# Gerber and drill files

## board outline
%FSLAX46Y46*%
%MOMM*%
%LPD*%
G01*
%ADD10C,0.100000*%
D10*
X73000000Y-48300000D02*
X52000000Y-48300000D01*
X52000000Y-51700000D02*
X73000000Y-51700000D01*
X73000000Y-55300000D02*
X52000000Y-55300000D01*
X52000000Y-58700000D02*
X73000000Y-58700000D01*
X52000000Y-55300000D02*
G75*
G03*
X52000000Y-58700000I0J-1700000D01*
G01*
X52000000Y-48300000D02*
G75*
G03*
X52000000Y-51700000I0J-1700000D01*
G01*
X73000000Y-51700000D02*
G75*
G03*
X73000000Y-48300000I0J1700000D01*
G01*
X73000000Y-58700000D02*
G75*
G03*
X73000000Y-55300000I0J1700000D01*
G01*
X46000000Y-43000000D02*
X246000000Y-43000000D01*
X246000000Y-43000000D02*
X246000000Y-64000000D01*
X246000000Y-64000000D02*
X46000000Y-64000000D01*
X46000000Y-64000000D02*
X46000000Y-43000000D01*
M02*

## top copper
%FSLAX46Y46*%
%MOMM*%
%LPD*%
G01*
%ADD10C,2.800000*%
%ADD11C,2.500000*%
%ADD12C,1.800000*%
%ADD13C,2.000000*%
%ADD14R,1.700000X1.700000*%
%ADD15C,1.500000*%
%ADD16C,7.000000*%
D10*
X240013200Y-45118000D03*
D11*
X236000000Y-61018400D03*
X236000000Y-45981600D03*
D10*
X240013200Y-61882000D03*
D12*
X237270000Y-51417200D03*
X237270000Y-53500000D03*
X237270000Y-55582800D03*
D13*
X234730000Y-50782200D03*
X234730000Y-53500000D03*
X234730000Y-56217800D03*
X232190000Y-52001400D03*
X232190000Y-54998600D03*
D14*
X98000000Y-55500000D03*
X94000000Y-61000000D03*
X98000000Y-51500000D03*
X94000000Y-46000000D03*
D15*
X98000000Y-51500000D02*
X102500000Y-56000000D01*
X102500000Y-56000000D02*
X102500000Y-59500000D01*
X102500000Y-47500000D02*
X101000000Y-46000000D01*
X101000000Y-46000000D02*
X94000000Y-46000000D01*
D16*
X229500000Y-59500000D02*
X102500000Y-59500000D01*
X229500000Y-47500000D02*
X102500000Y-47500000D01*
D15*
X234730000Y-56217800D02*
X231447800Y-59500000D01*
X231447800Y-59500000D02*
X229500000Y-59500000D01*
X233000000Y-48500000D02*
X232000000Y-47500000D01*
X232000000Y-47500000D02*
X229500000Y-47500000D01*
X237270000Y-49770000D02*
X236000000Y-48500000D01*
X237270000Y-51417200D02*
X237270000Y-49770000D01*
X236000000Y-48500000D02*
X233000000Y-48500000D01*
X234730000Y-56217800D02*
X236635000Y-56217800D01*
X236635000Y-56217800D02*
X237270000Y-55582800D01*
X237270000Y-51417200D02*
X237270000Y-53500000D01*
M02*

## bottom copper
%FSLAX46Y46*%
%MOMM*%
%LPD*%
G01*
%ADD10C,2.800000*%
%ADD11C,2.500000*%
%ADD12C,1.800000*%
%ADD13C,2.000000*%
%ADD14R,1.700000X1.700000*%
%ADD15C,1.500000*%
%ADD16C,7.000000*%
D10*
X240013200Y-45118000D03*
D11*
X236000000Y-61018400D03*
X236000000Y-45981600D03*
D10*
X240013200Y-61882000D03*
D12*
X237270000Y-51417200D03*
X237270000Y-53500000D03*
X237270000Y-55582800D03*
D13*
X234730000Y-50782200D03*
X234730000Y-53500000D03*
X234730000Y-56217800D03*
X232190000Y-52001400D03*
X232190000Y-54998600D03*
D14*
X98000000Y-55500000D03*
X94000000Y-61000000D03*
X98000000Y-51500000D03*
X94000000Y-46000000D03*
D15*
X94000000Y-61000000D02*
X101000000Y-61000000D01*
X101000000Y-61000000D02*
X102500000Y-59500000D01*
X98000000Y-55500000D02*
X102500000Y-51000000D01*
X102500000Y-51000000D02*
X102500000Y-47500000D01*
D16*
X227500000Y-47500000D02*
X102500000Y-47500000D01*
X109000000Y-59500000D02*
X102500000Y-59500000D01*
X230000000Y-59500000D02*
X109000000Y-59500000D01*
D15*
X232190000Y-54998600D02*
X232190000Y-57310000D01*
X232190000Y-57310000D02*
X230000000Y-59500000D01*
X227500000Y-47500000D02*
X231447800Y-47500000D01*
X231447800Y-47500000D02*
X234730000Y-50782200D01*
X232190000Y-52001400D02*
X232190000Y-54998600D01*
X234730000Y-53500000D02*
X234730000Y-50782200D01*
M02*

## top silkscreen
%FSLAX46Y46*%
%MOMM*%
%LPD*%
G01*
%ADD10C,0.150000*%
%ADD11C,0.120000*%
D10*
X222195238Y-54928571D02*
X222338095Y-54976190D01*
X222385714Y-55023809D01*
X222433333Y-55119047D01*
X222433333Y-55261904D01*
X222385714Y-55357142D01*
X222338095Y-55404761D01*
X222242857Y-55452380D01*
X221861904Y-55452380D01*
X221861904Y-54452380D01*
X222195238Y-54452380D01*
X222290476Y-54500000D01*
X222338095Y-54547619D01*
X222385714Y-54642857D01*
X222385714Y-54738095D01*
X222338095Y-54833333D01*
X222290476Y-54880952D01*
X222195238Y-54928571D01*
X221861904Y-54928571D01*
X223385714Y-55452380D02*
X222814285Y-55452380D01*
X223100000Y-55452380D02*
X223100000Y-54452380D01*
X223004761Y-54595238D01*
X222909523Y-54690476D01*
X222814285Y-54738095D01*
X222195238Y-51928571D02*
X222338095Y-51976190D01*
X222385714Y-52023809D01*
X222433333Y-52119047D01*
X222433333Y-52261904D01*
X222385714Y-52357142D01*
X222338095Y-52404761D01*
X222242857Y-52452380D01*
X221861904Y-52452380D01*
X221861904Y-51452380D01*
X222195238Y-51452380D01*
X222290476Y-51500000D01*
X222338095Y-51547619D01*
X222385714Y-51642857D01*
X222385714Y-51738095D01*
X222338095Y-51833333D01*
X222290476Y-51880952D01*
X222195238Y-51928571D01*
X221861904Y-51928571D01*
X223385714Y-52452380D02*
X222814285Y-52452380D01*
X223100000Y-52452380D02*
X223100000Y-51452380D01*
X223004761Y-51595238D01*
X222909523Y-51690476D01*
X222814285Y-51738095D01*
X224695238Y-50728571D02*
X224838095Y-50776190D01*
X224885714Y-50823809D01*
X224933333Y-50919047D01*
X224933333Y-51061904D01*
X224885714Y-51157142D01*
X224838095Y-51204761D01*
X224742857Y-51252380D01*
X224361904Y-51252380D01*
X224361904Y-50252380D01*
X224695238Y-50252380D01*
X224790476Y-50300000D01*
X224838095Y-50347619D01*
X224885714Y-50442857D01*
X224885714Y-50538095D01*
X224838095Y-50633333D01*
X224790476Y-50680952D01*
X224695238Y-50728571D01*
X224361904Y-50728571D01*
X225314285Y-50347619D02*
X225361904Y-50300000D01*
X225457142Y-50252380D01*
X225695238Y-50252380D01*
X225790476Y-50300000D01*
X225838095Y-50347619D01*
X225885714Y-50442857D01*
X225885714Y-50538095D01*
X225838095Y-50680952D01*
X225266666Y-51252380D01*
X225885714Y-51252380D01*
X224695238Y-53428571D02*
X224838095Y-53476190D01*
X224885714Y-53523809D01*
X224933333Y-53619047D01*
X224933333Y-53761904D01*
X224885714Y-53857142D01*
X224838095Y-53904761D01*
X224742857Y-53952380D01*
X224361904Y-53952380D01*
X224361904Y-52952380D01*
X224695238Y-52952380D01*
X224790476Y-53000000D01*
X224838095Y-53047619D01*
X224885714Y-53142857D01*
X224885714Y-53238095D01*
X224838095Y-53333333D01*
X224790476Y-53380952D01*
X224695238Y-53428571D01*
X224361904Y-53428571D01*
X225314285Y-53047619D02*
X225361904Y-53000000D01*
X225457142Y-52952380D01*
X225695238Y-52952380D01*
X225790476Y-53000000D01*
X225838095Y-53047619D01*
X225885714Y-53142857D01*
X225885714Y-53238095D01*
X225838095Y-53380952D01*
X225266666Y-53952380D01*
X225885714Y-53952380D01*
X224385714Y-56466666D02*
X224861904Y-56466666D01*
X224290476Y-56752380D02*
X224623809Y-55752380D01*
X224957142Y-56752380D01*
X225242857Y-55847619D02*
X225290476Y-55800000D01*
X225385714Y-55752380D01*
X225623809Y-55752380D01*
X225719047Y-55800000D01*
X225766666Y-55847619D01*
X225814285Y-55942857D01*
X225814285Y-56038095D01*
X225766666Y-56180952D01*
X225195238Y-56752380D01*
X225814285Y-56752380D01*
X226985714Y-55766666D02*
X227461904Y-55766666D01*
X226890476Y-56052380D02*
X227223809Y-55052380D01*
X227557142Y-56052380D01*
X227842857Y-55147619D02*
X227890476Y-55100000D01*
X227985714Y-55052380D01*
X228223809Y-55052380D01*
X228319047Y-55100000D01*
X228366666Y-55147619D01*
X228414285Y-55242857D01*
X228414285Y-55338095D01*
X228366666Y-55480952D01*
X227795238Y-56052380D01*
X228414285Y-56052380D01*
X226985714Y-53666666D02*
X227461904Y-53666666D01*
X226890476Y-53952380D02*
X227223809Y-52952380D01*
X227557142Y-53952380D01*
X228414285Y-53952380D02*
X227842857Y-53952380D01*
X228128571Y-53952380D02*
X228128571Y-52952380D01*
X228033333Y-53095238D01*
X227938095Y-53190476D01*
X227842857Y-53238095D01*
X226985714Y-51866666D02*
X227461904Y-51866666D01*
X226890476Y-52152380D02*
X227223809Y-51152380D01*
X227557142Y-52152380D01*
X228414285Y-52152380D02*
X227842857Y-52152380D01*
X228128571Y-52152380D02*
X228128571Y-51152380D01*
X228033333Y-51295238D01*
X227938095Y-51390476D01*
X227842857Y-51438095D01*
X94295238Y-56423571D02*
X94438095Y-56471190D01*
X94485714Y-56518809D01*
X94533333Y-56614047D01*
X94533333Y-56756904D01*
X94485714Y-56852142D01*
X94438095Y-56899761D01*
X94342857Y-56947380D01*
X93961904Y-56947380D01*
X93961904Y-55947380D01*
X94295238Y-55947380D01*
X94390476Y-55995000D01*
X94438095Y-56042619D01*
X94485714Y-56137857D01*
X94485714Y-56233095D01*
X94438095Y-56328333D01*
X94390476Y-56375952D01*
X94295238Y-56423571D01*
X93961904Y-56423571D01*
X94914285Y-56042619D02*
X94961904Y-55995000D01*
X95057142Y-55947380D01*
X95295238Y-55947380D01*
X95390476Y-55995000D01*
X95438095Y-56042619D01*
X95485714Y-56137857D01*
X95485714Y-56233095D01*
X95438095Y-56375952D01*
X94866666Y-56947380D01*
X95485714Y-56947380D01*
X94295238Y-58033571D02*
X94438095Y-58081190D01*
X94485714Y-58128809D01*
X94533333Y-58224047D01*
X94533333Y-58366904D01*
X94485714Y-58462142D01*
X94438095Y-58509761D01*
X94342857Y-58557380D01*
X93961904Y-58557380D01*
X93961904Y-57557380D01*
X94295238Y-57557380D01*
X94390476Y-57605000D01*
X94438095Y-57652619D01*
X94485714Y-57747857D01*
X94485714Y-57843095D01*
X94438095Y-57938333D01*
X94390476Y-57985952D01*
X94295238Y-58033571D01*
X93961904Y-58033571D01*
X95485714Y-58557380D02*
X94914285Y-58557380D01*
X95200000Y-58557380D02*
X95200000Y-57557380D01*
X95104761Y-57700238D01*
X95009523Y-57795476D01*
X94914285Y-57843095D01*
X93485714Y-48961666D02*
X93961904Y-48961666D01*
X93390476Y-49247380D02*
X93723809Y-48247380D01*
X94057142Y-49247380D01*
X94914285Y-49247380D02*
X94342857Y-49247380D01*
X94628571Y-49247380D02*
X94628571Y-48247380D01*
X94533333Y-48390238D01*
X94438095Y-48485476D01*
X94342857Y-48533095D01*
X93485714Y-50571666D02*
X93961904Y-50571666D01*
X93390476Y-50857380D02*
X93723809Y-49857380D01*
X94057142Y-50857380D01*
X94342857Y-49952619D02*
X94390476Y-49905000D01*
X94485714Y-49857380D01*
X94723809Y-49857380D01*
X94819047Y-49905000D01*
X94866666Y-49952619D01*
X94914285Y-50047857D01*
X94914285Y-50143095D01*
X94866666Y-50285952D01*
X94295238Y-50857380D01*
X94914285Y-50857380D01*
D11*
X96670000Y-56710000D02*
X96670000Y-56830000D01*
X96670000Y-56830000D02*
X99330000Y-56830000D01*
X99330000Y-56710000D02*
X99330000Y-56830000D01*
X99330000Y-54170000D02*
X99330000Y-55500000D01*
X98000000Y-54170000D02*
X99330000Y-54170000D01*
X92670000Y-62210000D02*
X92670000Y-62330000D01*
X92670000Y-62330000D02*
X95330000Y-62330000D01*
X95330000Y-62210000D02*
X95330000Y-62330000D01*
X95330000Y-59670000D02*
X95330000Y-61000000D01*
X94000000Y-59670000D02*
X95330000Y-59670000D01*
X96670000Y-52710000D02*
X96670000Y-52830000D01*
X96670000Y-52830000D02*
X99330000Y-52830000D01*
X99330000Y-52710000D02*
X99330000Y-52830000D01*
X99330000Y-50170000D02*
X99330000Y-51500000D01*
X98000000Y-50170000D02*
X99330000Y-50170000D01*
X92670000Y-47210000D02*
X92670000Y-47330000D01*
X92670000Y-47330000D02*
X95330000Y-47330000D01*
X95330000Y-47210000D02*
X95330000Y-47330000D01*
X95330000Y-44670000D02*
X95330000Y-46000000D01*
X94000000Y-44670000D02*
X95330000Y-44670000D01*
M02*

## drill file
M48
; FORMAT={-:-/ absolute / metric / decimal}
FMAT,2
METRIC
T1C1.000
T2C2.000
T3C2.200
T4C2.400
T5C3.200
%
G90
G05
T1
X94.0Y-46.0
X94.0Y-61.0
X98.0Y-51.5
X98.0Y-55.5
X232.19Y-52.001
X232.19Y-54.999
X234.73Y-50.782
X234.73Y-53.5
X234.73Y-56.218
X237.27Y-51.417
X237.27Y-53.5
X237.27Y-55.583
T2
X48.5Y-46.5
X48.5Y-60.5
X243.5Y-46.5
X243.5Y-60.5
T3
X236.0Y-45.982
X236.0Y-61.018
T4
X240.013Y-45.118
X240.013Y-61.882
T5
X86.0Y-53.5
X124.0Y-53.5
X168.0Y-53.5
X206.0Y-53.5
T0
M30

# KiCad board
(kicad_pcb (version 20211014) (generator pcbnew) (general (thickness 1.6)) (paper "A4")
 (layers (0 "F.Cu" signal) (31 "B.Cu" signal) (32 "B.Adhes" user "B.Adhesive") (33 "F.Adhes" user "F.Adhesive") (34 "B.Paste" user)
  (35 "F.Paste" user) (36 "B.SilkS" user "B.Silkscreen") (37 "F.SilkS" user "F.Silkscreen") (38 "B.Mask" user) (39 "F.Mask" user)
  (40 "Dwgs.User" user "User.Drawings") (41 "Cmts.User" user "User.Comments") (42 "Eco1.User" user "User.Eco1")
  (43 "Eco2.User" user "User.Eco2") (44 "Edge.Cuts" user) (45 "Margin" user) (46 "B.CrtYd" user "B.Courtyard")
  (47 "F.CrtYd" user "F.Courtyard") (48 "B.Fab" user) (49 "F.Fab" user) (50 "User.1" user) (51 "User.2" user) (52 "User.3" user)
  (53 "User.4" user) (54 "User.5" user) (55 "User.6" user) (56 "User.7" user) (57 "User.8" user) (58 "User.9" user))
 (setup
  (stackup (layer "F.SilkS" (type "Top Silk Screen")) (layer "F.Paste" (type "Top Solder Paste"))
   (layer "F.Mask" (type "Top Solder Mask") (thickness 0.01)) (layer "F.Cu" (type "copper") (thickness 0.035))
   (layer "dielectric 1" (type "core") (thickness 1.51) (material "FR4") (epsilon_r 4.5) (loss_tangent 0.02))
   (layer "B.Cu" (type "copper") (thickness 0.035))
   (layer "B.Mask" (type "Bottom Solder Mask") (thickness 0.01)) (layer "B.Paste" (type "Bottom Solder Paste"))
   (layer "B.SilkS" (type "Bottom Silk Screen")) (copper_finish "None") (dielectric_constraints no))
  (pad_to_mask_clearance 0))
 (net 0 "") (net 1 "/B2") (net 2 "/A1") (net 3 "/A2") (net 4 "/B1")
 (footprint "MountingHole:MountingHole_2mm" (layer "F.Cu") (at 243.5 46.5)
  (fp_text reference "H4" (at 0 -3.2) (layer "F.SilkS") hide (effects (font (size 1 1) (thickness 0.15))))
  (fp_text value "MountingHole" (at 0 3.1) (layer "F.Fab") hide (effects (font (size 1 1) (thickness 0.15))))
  (pad "" np_thru_hole circle (at 0 0) (size 2 2) (drill 2) (layers *.Cu *.Mask)))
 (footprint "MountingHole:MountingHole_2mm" (layer "F.Cu") (at 48.5 60.5)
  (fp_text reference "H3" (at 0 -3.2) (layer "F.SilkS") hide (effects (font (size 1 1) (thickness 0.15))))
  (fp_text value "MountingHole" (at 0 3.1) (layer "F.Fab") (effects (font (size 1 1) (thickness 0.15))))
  (pad "" np_thru_hole circle (at 0 0) (size 2 2) (drill 2) (layers *.Cu *.Mask)))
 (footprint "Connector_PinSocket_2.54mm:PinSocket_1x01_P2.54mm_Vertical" (layer "F.Cu") (at 98 55.5)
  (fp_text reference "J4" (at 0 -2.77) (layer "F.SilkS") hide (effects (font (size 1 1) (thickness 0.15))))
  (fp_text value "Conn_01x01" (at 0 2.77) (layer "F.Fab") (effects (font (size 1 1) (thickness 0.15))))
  (fp_line (start -1.33 1.21) (end -1.33 1.33) (layer "F.SilkS") (width 0.12))
  (fp_line (start 0 -1.33) (end 1.33 -1.33) (layer "F.SilkS") (width 0.12))
  (fp_line (start 1.33 1.21) (end 1.33 1.33) (layer "F.SilkS") (width 0.12))
  (fp_line (start 1.33 -1.33) (end 1.33 0) (layer "F.SilkS") (width 0.12))
  (fp_line (start -1.33 1.33) (end 1.33 1.33) (layer "F.SilkS") (width 0.12))
  (pad "1" thru_hole rect (at 0 0) (size 1.7 1.7) (drill 1) (layers *.Cu *.Mask) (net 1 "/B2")))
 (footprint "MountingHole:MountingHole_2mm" (layer "F.Cu") (at 48.5 46.5)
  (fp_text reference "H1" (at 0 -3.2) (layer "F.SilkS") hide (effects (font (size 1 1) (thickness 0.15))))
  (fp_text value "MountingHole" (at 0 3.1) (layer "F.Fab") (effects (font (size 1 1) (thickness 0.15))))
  (pad "" np_thru_hole circle (at 0 0) (size 2 2) (drill 2) (layers *.Cu *.Mask)))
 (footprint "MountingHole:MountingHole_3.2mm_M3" (layer "F.Cu") (at 168 53.5)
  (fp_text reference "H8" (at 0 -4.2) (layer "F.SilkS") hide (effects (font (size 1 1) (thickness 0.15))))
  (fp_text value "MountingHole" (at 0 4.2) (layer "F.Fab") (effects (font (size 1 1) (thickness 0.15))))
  (pad "" np_thru_hole circle (at 0 0) (size 3.2 3.2) (drill 3.2) (layers *.Cu *.Mask)))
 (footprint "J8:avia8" (layer "F.Cu") (at 234.73 53.5 -90)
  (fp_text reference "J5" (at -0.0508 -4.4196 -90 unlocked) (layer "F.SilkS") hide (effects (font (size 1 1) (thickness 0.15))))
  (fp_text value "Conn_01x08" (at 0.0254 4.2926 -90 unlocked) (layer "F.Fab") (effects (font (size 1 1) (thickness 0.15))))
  (pad "" np_thru_hole circle (at -8.382 -5.2832 270) (size 2.8 2.8) (drill 2.4) (layers F&B.Cu *.Mask))
  (pad "" np_thru_hole circle (at 7.5184 -1.27 270) (size 2.5 2.5) (drill 2.2) (layers F&B.Cu *.Mask))
  (pad "" np_thru_hole circle (at -7.5184 -1.27 270) (size 2.5 2.5) (drill 2.2) (layers F&B.Cu *.Mask))
  (pad "" np_thru_hole circle (at 8.382 -5.2832 270) (size 2.8 2.8) (drill 2.4) (layers F&B.Cu *.Mask))
  (pad "1" thru_hole circle (at -2.0828 -2.54 270) (size 1.8 1.8) (drill 1) (layers *.Cu *.Mask) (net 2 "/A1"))
  (pad "2" thru_hole circle (at 0 -2.54 270) (size 1.8 1.8) (drill 1) (layers *.Cu *.Mask) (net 2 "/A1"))
  (pad "3" thru_hole circle (at 2.0828 -2.54 270) (size 1.8 1.8) (drill 1) (layers *.Cu *.Mask) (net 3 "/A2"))
  (pad "4" thru_hole circle (at -2.7178 0 270) (size 2 2) (drill 1) (layers *.Cu *.Mask) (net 1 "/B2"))
  (pad "5" thru_hole circle (at 0 0 270) (size 2 2) (drill 1) (layers *.Cu *.Mask) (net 1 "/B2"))
  (pad "6" thru_hole circle (at 2.7178 0 270) (size 2 2) (drill 1) (layers *.Cu *.Mask) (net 3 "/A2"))
  (pad "7" thru_hole circle (at -1.4986 2.54 270) (size 2 2) (drill 1) (layers *.Cu *.Mask) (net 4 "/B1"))
  (pad "8" thru_hole circle (at 1.4986 2.54 270) (size 2 2) (drill 1) (layers *.Cu *.Mask) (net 4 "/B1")))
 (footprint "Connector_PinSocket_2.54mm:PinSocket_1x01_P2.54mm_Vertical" (layer "F.Cu") (at 94 46)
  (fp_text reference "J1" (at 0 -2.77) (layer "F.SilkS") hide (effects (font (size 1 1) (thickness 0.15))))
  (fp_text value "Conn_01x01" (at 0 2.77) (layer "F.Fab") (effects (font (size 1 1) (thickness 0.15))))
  (fp_line (start 0 -1.33) (end 1.33 -1.33) (layer "F.SilkS") (width 0.12))
  (fp_line (start 1.33 1.21) (end 1.33 1.33) (layer "F.SilkS") (width 0.12))
  (fp_line (start -1.33 1.21) (end -1.33 1.33) (layer "F.SilkS") (width 0.12))
  (fp_line (start 1.33 -1.33) (end 1.33 0) (layer "F.SilkS") (width 0.12))
  (fp_line (start -1.33 1.33) (end 1.33 1.33) (layer "F.SilkS") (width 0.12))
  (pad "1" thru_hole rect (at 0 0) (size 1.7 1.7) (drill 1) (layers *.Cu *.Mask) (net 2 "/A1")))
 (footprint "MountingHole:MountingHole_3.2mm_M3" (layer "F.Cu") (at 124 53.5)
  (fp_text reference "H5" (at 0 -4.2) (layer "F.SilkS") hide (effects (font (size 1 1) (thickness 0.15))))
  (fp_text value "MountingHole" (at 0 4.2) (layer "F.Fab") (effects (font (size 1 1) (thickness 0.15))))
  (pad "" np_thru_hole circle (at 0 0) (size 3.2 3.2) (drill 3.2) (layers *.Cu *.Mask)))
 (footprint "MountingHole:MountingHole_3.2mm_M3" (layer "F.Cu") (at 86 53.5)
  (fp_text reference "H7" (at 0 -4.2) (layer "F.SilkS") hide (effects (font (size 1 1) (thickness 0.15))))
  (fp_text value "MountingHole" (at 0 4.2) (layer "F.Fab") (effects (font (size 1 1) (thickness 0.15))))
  (pad "" np_thru_hole circle (at 0 0) (size 3.2 3.2) (drill 3.2) (layers *.Cu *.Mask)))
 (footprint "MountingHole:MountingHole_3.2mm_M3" (layer "F.Cu") (at 206 53.5)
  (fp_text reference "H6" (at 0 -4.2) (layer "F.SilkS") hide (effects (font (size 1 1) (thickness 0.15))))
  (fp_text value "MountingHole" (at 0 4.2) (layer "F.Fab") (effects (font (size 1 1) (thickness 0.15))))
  (pad "" np_thru_hole circle (at 0 0) (size 3.2 3.2) (drill 3.2) (layers *.Cu *.Mask)))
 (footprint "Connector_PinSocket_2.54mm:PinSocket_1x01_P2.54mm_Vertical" (layer "F.Cu") (at 94 61)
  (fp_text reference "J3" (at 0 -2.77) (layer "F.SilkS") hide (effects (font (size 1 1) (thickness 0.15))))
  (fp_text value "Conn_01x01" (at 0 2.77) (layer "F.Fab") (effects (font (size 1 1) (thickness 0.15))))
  (fp_line (start -1.33 1.33) (end 1.33 1.33) (layer "F.SilkS") (width 0.12))
  (fp_line (start 1.33 -1.33) (end 1.33 0) (layer "F.SilkS") (width 0.12))
  (fp_line (start -1.33 1.21) (end -1.33 1.33) (layer "F.SilkS") (width 0.12))
  (fp_line (start 1.33 1.21) (end 1.33 1.33) (layer "F.SilkS") (width 0.12))
  (fp_line (start 0 -1.33) (end 1.33 -1.33) (layer "F.SilkS") (width 0.12))
  (pad "1" thru_hole rect (at 0 0) (size 1.7 1.7) (drill 1) (layers *.Cu *.Mask) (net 4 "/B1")))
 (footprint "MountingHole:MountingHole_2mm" (layer "F.Cu") (at 243.5 60.5)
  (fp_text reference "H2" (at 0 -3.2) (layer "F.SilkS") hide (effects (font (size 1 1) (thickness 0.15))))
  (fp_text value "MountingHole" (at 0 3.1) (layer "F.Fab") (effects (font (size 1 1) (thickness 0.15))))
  (pad "" np_thru_hole circle (at 0 0) (size 2 2) (drill 2) (layers *.Cu *.Mask)))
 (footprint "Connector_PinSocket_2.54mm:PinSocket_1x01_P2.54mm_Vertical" (layer "F.Cu") (at 98 51.5)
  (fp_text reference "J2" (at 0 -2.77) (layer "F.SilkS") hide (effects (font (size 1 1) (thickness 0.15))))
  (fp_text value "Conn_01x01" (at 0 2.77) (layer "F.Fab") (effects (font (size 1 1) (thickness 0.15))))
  (fp_line (start 0 -1.33) (end 1.33 -1.33) (layer "F.SilkS") (width 0.12))
  (fp_line (start 1.33 -1.33) (end 1.33 0) (layer "F.SilkS") (width 0.12))
  (fp_line (start -1.33 1.21) (end -1.33 1.33) (layer "F.SilkS") (width 0.12))
  (fp_line (start 1.33 1.21) (end 1.33 1.33) (layer "F.SilkS") (width 0.12))
  (fp_line (start -1.33 1.33) (end 1.33 1.33) (layer "F.SilkS") (width 0.12))
  (pad "1" thru_hole rect (at 0 0) (size 1.7 1.7) (drill 1) (layers *.Cu *.Mask) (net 3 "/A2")))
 (gr_line (start 52 58.7) (end 73 58.7) (layer "Edge.Cuts") (width 0.1))
 (gr_line (start 52 51.7) (end 73 51.7) (layer "Edge.Cuts") (width 0.1))
 (gr_arc (start 52 58.7) (mid 50.3 57) (end 52 55.3) (layer "Edge.Cuts") (width 0.1))
 (gr_arc (start 52 51.7) (mid 50.3 50) (end 52 48.3) (layer "Edge.Cuts") (width 0.1))
 (gr_line (start 73 55.3) (end 52 55.3) (layer "Edge.Cuts") (width 0.1))
 (gr_rect (start 46 43) (end 246 64) (layer "Edge.Cuts") (width 0.1) (fill none))
 (gr_arc (start 73 48.3) (mid 74.7 50) (end 73 51.7) (layer "Edge.Cuts") (width 0.1))
 (gr_arc (start 73 55.3) (mid 74.7 57) (end 73 58.7) (layer "Edge.Cuts") (width 0.1))
 (gr_line (start 73 48.3) (end 52 48.3) (layer "Edge.Cuts") (width 0.1))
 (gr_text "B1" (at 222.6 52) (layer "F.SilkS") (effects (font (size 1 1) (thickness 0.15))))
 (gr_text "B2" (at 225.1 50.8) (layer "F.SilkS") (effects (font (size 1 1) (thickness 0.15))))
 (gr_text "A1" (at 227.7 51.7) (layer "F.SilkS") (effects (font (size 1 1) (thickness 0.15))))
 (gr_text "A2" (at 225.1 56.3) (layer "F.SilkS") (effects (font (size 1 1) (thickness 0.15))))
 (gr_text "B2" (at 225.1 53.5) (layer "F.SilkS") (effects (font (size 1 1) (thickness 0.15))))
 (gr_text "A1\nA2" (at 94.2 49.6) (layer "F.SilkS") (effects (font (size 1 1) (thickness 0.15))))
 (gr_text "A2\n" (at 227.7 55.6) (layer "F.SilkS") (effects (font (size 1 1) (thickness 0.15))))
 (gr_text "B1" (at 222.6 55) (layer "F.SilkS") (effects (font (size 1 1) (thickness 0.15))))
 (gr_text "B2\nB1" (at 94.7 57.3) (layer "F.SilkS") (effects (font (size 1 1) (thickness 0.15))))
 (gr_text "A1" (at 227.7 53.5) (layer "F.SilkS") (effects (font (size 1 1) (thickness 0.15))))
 (segment (start 237.27 51.4172) (end 237.27 49.77) (width 1.5) (layer "F.Cu") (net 2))
 (segment (start 102.5 47.5) (end 101 46) (width 1.5) (layer "F.Cu") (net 2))
 (segment (start 232 47.5) (end 229.5 47.5) (width 1.5) (layer "F.Cu") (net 2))
 (segment (start 236 48.5) (end 233 48.5) (width 1.5) (layer "F.Cu") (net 2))
 (segment (start 229.5 47.5) (end 102.5 47.5) (width 7) (layer "F.Cu") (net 2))
 (segment (start 237.27 49.77) (end 236 48.5) (width 1.5) (layer "F.Cu") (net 2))
 (segment (start 233 48.5) (end 232 47.5) (width 1.5) (layer "F.Cu") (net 2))
 (segment (start 101 46) (end 94 46) (width 1.5) (layer "F.Cu") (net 2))
 (segment (start 237.27 51.4172) (end 237.27 53.5) (width 1.5) (layer "F.Cu") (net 2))
 (segment (start 231.4478 59.5) (end 229.5 59.5) (width 1.5) (layer "F.Cu") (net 3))
 (segment (start 234.73 56.2178) (end 231.4478 59.5) (width 1.5) (layer "F.Cu") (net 3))
 (segment (start 236.635 56.2178) (end 237.27 55.5828) (width 1.5) (layer "F.Cu") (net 3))
 (segment (start 102.5 56) (end 102.5 59.5) (width 1.5) (layer "F.Cu") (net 3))
 (segment (start 98 51.5) (end 102.5 56) (width 1.5) (layer "F.Cu") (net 3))
 (segment (start 229.5 59.5) (end 102.5 59.5) (width 7) (layer "F.Cu") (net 3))
 (segment (start 234.73 56.2178) (end 236.635 56.2178) (width 1.5) (layer "F.Cu") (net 3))
 (segment (start 232.19 52.0014) (end 232.19 54.9986) (width 1.5) (layer "B.Cu") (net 4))
 (segment (start 109 59.5) (end 102.5 59.5) (width 7) (layer "B.Cu") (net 4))
 (segment (start 232.19 57.31) (end 230 59.5) (width 1.5) (layer "B.Cu") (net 4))
 (segment (start 230 59.5) (end 109 59.5) (width 7) (layer "B.Cu") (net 4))
 (segment (start 232.19 54.9986) (end 232.19 57.31) (width 1.5) (layer "B.Cu") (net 4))
 (segment (start 101 61) (end 102.5 59.5) (width 1.5) (layer "B.Cu") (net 4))
 (segment (start 94 61) (end 101 61) (width 1.5) (layer "B.Cu") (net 4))
 (segment (start 102.5 51) (end 102.5 47.5) (width 1.5) (layer "B.Cu") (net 1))
 (segment (start 227.5 47.5) (end 102.5 47.5) (width 7) (layer "B.Cu") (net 1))
 (segment (start 234.73 53.5) (end 234.73 50.7822) (width 1.5) (layer "B.Cu") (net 1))
 (segment (start 227.5 47.5) (end 231.4478 47.5) (width 1.5) (layer "B.Cu") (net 1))
 (segment (start 98 55.5) (end 102.5 51) (width 1.5) (layer "B.Cu") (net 1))
 (segment (start 231.4478 47.5) (end 234.73 50.7822) (width 1.5) (layer "B.Cu") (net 1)))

